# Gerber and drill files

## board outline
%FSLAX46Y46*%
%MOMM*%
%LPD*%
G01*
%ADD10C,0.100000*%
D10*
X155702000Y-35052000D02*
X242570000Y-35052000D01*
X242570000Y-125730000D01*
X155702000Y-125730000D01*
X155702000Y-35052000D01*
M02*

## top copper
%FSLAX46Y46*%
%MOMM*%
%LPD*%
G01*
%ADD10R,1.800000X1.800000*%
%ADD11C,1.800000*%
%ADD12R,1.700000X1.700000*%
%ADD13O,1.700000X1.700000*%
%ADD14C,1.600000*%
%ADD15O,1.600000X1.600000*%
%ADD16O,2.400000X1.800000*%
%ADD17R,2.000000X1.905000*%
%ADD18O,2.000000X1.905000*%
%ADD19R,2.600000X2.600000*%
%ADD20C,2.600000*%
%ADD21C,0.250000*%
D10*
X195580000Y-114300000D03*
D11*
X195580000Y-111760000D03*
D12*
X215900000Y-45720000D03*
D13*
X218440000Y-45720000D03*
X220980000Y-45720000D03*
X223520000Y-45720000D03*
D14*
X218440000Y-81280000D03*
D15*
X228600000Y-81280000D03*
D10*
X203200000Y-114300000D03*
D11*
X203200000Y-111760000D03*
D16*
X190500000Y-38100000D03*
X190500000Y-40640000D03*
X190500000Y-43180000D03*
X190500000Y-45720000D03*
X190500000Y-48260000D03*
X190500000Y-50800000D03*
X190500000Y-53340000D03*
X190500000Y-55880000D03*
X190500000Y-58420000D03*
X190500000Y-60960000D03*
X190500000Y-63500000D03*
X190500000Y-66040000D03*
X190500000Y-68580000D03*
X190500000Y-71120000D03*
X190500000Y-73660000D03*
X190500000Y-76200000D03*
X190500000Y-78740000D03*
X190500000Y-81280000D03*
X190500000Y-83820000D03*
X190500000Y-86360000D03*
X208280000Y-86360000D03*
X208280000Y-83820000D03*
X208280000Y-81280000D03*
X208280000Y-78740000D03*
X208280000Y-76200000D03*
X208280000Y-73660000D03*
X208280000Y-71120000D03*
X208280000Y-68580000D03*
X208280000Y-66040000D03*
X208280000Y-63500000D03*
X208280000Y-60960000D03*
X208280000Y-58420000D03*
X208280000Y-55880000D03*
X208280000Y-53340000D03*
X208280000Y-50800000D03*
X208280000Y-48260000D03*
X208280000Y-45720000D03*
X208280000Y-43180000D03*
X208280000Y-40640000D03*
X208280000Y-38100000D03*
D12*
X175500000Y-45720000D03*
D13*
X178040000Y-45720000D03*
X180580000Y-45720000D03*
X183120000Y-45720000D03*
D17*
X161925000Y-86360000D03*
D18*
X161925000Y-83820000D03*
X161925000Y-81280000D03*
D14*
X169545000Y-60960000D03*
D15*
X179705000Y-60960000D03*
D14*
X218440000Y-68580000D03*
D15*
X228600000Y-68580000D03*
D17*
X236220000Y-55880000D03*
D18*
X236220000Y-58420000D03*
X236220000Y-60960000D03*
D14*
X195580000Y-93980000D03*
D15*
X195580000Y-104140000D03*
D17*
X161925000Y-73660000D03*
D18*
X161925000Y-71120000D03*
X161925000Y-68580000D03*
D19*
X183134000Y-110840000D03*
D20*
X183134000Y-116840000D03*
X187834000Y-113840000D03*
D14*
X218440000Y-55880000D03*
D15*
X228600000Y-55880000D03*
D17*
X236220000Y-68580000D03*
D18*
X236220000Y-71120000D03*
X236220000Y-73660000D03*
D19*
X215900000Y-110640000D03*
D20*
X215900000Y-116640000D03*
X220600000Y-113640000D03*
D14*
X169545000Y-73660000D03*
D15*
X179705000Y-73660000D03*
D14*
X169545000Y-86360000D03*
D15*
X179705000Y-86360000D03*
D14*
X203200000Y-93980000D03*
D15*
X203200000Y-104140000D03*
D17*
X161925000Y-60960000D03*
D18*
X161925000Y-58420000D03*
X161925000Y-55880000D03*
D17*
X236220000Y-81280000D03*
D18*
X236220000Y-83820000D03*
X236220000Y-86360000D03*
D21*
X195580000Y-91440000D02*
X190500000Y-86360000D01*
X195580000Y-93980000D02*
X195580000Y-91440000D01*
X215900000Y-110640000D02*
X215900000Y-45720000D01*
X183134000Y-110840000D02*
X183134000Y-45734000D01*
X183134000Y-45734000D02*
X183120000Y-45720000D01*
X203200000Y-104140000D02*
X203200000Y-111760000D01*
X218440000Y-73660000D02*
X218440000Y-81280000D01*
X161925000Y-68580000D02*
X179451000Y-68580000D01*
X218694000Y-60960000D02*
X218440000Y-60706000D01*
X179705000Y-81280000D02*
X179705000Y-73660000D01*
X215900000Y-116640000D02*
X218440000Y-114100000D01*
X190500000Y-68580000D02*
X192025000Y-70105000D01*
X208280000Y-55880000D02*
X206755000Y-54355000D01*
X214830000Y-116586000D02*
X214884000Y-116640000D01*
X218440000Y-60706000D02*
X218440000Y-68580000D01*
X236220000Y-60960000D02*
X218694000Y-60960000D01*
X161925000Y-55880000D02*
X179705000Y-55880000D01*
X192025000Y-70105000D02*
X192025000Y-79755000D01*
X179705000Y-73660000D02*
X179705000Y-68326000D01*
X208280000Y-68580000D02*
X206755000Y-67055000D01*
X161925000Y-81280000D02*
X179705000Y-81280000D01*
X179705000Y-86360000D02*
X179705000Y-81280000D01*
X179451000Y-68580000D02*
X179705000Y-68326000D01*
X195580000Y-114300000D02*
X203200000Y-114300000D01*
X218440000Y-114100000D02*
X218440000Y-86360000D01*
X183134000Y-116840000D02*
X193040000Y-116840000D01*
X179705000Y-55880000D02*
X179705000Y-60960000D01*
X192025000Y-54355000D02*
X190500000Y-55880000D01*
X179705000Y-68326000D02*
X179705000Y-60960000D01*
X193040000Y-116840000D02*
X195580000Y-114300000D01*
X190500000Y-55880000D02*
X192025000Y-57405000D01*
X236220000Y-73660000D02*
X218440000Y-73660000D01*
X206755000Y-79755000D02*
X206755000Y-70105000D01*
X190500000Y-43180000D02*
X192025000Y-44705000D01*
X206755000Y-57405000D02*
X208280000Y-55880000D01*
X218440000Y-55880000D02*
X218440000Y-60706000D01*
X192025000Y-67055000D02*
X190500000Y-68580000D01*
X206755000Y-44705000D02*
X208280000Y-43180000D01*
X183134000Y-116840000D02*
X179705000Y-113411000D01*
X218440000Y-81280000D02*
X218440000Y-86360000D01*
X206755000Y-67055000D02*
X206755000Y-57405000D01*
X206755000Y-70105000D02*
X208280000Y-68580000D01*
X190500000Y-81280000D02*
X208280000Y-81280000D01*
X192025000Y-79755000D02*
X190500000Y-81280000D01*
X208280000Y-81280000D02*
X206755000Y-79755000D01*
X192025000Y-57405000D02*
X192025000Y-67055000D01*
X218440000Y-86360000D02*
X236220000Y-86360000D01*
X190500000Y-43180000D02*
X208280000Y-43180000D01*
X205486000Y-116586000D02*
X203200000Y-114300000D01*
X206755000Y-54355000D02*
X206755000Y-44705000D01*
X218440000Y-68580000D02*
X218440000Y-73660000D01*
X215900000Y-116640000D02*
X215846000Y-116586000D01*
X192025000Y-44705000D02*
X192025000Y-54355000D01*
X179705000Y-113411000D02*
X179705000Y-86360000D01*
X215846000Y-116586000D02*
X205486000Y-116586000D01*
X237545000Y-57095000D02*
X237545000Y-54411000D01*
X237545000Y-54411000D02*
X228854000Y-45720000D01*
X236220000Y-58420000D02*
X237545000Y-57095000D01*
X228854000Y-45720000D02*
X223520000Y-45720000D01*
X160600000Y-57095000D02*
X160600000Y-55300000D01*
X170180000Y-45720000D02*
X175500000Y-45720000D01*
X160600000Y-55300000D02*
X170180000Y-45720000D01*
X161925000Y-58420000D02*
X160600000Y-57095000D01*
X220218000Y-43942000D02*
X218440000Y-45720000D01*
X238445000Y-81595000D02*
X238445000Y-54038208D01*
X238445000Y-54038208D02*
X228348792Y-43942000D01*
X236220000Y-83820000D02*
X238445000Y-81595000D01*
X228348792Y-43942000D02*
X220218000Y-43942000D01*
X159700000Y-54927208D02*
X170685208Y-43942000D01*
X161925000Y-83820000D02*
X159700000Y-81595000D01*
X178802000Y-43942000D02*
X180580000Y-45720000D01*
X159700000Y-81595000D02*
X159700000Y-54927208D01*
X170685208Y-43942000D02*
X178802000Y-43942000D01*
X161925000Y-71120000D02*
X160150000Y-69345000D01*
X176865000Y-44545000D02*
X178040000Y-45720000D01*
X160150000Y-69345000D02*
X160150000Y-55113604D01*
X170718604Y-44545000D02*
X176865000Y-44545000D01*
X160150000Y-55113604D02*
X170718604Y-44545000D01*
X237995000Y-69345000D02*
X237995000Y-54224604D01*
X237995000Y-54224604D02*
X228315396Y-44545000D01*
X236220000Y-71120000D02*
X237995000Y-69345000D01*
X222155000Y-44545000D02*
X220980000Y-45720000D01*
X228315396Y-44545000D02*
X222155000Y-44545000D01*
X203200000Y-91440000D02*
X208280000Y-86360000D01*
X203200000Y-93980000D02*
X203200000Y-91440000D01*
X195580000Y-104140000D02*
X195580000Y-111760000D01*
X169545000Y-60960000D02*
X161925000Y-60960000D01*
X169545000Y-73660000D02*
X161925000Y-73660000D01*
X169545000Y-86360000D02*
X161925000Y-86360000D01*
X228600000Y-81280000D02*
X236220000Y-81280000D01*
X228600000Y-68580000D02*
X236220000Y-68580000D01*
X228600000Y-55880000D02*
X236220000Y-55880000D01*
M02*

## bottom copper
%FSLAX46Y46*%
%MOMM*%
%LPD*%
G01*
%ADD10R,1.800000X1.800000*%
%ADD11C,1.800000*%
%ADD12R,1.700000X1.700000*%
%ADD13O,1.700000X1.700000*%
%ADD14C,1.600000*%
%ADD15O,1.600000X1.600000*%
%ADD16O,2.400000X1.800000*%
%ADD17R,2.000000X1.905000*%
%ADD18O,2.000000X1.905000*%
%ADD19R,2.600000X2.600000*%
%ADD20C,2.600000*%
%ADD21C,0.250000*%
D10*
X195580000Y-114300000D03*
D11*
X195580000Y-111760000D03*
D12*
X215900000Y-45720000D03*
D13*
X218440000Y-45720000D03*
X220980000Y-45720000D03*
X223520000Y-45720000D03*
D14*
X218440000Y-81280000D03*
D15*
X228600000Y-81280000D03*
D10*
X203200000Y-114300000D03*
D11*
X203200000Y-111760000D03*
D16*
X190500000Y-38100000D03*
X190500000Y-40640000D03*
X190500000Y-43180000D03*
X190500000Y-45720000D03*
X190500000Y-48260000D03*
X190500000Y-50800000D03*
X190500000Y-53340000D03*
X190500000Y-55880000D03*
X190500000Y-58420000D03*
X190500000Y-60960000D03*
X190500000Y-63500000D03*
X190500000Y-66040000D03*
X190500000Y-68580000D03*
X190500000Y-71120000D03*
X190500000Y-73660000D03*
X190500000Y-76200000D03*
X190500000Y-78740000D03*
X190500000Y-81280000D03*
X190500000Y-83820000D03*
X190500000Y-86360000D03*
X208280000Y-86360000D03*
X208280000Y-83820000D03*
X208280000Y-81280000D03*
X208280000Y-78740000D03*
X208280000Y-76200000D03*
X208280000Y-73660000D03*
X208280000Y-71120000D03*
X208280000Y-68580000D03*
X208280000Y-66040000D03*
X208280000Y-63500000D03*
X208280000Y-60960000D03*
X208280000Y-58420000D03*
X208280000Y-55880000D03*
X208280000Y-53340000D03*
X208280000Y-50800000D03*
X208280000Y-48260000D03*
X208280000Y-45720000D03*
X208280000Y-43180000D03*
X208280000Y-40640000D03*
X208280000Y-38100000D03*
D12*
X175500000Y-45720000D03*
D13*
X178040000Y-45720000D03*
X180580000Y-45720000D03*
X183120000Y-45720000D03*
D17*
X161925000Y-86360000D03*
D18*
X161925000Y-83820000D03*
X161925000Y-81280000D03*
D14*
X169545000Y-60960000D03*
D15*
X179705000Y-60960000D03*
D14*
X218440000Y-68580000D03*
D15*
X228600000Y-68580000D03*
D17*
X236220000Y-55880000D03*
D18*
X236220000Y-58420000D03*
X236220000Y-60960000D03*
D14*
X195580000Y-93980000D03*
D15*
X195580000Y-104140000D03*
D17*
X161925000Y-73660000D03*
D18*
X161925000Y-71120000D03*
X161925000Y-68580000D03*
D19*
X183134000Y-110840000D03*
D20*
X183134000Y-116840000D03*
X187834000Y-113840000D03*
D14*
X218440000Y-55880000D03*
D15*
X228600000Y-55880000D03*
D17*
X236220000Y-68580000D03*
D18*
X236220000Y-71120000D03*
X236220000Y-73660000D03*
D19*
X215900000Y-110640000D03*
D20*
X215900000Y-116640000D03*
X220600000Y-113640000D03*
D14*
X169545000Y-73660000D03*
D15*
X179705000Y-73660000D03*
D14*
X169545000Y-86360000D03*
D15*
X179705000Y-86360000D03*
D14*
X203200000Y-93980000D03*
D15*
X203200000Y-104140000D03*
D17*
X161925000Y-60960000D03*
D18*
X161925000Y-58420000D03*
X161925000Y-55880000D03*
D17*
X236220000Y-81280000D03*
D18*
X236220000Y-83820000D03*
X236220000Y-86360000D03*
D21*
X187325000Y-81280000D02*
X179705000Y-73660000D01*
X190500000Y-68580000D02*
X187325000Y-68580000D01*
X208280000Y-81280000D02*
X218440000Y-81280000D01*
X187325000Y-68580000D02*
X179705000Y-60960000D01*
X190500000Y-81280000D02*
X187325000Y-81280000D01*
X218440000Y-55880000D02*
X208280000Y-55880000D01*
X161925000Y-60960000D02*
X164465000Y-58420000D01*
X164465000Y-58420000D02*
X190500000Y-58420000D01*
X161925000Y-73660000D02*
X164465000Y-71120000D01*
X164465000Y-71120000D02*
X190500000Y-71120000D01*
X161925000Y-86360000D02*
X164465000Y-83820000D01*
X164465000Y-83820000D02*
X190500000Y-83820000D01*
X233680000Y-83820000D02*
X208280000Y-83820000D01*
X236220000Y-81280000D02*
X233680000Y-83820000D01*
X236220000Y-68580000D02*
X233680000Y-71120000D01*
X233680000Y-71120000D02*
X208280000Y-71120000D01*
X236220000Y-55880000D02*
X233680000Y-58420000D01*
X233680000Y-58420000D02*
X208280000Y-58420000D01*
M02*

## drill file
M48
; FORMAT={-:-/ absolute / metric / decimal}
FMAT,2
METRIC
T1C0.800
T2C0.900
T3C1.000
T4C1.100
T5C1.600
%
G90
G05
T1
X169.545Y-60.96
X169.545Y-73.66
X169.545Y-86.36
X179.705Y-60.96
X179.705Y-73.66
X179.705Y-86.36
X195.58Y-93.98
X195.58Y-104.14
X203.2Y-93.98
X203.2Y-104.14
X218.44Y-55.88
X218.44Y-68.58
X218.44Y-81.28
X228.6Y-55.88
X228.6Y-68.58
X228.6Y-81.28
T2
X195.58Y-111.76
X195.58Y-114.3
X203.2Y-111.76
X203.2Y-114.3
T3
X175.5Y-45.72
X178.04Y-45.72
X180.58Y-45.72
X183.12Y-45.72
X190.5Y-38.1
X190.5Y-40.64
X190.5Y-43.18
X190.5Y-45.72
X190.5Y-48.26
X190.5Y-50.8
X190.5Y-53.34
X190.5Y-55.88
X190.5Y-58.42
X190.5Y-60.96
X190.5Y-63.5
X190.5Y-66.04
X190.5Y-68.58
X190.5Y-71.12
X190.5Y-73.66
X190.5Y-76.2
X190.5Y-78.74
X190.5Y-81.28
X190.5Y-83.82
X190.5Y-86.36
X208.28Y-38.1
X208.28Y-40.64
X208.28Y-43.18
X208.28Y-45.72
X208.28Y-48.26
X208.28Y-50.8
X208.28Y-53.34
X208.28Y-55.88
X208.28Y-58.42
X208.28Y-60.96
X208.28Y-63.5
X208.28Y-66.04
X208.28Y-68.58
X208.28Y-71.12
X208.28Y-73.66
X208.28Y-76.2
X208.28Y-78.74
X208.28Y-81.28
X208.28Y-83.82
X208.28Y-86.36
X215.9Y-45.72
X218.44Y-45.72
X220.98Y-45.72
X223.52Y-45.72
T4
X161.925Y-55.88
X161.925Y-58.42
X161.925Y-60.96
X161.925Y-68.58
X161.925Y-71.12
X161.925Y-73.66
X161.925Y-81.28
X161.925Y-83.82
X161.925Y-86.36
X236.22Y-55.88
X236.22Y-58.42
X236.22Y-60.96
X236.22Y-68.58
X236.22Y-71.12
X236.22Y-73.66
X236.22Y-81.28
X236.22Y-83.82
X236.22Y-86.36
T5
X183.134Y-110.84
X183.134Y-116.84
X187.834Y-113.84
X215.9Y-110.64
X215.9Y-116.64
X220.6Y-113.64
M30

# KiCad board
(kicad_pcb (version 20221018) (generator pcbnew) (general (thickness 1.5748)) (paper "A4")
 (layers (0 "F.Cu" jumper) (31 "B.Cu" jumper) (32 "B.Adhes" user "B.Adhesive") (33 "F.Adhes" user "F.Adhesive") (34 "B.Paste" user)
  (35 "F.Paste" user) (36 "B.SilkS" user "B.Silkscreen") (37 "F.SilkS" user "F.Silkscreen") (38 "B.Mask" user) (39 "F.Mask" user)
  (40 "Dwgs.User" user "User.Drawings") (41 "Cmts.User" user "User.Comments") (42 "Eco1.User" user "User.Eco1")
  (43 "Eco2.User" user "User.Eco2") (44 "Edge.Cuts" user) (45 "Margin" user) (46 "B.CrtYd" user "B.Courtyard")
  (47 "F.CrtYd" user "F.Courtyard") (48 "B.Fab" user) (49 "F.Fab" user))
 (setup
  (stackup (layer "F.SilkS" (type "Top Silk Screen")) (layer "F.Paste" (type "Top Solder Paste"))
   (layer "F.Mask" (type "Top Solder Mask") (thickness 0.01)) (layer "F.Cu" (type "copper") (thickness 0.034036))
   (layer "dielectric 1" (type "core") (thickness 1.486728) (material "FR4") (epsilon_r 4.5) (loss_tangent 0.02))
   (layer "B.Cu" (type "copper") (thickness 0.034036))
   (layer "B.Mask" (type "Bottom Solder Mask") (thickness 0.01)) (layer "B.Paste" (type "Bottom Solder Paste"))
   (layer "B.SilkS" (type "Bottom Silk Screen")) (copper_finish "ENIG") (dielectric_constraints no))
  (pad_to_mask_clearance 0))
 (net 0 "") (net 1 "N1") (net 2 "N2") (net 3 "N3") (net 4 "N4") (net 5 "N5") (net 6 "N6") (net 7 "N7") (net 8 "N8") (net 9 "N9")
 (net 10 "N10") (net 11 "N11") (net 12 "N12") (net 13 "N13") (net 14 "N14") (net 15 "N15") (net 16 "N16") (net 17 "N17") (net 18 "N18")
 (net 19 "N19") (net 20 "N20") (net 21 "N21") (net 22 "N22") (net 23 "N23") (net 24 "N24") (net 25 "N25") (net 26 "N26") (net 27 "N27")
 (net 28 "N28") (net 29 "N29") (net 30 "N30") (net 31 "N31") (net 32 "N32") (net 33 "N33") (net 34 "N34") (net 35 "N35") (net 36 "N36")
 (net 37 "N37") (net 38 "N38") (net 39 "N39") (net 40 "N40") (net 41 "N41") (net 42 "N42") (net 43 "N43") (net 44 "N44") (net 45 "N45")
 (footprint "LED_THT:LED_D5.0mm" (layer "F.Cu") (at 195.58 114.3 90)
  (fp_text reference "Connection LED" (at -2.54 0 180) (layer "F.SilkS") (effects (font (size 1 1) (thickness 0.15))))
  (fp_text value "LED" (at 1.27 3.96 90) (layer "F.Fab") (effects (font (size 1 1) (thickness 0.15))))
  (pad "1" thru_hole rect (at 0 0 90) (size 1.8 1.8) (drill 0.9) (layers "*.Cu" "*.Mask") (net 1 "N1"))
  (pad "2" thru_hole circle (at 2.54 0 90) (size 1.8 1.8) (drill 0.9) (layers "*.Cu" "*.Mask") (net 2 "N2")))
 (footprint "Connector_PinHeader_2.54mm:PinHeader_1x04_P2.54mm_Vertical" (layer "F.Cu") (at 215.9 45.72 90)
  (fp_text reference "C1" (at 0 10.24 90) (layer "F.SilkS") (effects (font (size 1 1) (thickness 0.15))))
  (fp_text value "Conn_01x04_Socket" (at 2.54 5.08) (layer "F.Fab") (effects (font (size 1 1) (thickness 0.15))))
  (pad "1" thru_hole rect (at 0 0 90) (size 1.7 1.7) (drill 1) (layers "*.Cu" "*.Mask") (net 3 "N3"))
  (pad "2" thru_hole oval (at 0 2.54 90) (size 1.7 1.7) (drill 1) (layers "*.Cu" "*.Mask") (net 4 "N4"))
  (pad "3" thru_hole oval (at 0 5.08 90) (size 1.7 1.7) (drill 1) (layers "*.Cu" "*.Mask") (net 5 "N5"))
  (pad "4" thru_hole oval (at 0 7.62 90) (size 1.7 1.7) (drill 1) (layers "*.Cu" "*.Mask") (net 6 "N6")))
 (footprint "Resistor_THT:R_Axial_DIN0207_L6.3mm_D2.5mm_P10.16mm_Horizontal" (layer "F.Cu") (at 218.44 81.28)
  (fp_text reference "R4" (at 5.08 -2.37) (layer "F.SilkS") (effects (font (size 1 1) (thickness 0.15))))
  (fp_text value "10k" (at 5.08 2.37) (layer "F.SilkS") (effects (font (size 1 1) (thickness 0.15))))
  (pad "1" thru_hole circle (at 0 0) (size 1.6 1.6) (drill 0.8) (layers "*.Cu" "*.Mask") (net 1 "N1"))
  (pad "2" thru_hole oval (at 10.16 0) (size 1.6 1.6) (drill 0.8) (layers "*.Cu" "*.Mask") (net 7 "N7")))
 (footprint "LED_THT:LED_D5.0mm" (layer "F.Cu") (at 203.2 114.3 90)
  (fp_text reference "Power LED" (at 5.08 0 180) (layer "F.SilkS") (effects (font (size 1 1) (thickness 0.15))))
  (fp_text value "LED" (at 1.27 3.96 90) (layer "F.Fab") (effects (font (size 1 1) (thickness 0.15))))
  (pad "1" thru_hole rect (at 0 0 90) (size 1.8 1.8) (drill 0.9) (layers "*.Cu" "*.Mask") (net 1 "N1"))
  (pad "2" thru_hole circle (at 2.54 0 90) (size 1.8 1.8) (drill 0.9) (layers "*.Cu" "*.Mask") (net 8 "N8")))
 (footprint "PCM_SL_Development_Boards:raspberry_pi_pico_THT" (layer "F.Cu") (at 190.5 38.1)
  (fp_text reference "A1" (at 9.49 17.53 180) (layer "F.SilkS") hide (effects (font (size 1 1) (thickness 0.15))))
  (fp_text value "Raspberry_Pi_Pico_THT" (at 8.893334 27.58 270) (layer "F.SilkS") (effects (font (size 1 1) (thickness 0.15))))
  (pad "1" thru_hole oval (at 0 0 270) (size 1.8 2.4) (drill 1) (layers "*.Cu" "*.Mask") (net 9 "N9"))
  (pad "2" thru_hole oval (at 0 2.54 270) (size 1.8 2.4) (drill 1) (layers "*.Cu" "*.Mask") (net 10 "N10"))
  (pad "3" thru_hole oval (at 0 5.08 270) (size 1.8 2.4) (drill 1) (layers "*.Cu" "*.Mask") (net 1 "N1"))
  (pad "4" thru_hole oval (at 0 7.62 270) (size 1.8 2.4) (drill 1) (layers "*.Cu" "*.Mask") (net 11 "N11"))
  (pad "5" thru_hole oval (at 0 10.16 270) (size 1.8 2.4) (drill 1) (layers "*.Cu" "*.Mask") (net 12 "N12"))
  (pad "6" thru_hole oval (at 0 12.7 270) (size 1.8 2.4) (drill 1) (layers "*.Cu" "*.Mask") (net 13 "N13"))
  (pad "7" thru_hole oval (at 0 15.24 270) (size 1.8 2.4) (drill 1) (layers "*.Cu" "*.Mask") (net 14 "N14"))
  (pad "8" thru_hole oval (at 0 17.78 270) (size 1.8 2.4) (drill 1) (layers "*.Cu" "*.Mask") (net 1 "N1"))
  (pad "9" thru_hole oval (at 0 20.32 270) (size 1.8 2.4) (drill 1) (layers "*.Cu" "*.Mask") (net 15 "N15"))
  (pad "10" thru_hole oval (at 0 22.86 270) (size 1.8 2.4) (drill 1) (layers "*.Cu" "*.Mask") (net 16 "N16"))
  (pad "11" thru_hole oval (at 0 25.4 270) (size 1.8 2.4) (drill 1) (layers "*.Cu" "*.Mask") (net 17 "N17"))
  (pad "12" thru_hole oval (at 0 27.94 270) (size 1.8 2.4) (drill 1) (layers "*.Cu" "*.Mask") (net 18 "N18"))
  (pad "13" thru_hole oval (at 0 30.48 270) (size 1.8 2.4) (drill 1) (layers "*.Cu" "*.Mask") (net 1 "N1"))
  (pad "14" thru_hole oval (at 0 33.02 270) (size 1.8 2.4) (drill 1) (layers "*.Cu" "*.Mask") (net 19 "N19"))
  (pad "15" thru_hole oval (at 0 35.56 270) (size 1.8 2.4) (drill 1) (layers "*.Cu" "*.Mask") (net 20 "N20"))
  (pad "16" thru_hole oval (at 0 38.1 270) (size 1.8 2.4) (drill 1) (layers "*.Cu" "*.Mask") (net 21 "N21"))
  (pad "17" thru_hole oval (at 0 40.64 270) (size 1.8 2.4) (drill 1) (layers "*.Cu" "*.Mask") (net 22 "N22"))
  (pad "18" thru_hole oval (at 0 43.18 270) (size 1.8 2.4) (drill 1) (layers "*.Cu" "*.Mask") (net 1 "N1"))
  (pad "19" thru_hole oval (at 0 45.72 270) (size 1.8 2.4) (drill 1) (layers "*.Cu" "*.Mask") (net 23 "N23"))
  (pad "20" thru_hole oval (at 0 48.26 270) (size 1.8 2.4) (drill 1) (layers "*.Cu" "*.Mask") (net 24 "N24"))
  (pad "21" thru_hole oval (at 17.78 48.26 270) (size 1.8 2.4) (drill 1) (layers "*.Cu" "*.Mask") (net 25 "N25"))
  (pad "22" thru_hole oval (at 17.78 45.72 270) (size 1.8 2.4) (drill 1) (layers "*.Cu" "*.Mask") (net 7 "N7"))
  (pad "23" thru_hole oval (at 17.78 43.18 270) (size 1.8 2.4) (drill 1) (layers "*.Cu" "*.Mask") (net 1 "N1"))
  (pad "24" thru_hole oval (at 17.78 40.64 270) (size 1.8 2.4) (drill 1) (layers "*.Cu" "*.Mask") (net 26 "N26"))
  (pad "25" thru_hole oval (at 17.78 38.1 270) (size 1.8 2.4) (drill 1) (layers "*.Cu" "*.Mask") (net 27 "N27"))
  (pad "26" thru_hole oval (at 17.78 35.56 270) (size 1.8 2.4) (drill 1) (layers "*.Cu" "*.Mask") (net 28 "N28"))
  (pad "27" thru_hole oval (at 17.78 33.02 270) (size 1.8 2.4) (drill 1) (layers "*.Cu" "*.Mask") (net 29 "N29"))
  (pad "28" thru_hole oval (at 17.78 30.48 270) (size 1.8 2.4) (drill 1) (layers "*.Cu" "*.Mask") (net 1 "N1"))
  (pad "29" thru_hole oval (at 17.78 27.94 270) (size 1.8 2.4) (drill 1) (layers "*.Cu" "*.Mask") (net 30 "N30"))
  (pad "30" thru_hole oval (at 17.78 25.4 270) (size 1.8 2.4) (drill 1) (layers "*.Cu" "*.Mask") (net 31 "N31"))
  (pad "31" thru_hole oval (at 17.78 22.86 270) (size 1.8 2.4) (drill 1) (layers "*.Cu" "*.Mask") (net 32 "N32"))
  (pad "32" thru_hole oval (at 17.78 20.32 270) (size 1.8 2.4) (drill 1) (layers "*.Cu" "*.Mask") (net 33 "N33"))
  (pad "33" thru_hole oval (at 17.78 17.78 270) (size 1.8 2.4) (drill 1) (layers "*.Cu" "*.Mask") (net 1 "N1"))
  (pad "34" thru_hole oval (at 17.78 15.24 270) (size 1.8 2.4) (drill 1) (layers "*.Cu" "*.Mask") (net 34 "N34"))
  (pad "35" thru_hole oval (at 17.78 12.7 270) (size 1.8 2.4) (drill 1) (layers "*.Cu" "*.Mask") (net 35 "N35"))
  (pad "36" thru_hole oval (at 17.78 10.16 270) (size 1.8 2.4) (drill 1) (layers "*.Cu" "*.Mask") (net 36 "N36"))
  (pad "37" thru_hole oval (at 17.78 7.62 270) (size 1.8 2.4) (drill 1) (layers "*.Cu" "*.Mask") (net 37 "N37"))
  (pad "38" thru_hole oval (at 17.78 5.08 270) (size 1.8 2.4) (drill 1) (layers "*.Cu" "*.Mask") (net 1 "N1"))
  (pad "39" thru_hole oval (at 17.78 2.54 270) (size 1.8 2.4) (drill 1) (layers "*.Cu" "*.Mask") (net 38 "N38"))
  (pad "40" thru_hole oval (at 17.78 0 270) (size 1.8 2.4) (drill 1) (layers "*.Cu" "*.Mask") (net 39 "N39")))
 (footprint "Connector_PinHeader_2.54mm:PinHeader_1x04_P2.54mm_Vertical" (layer "F.Cu") (at 175.5 45.72 90)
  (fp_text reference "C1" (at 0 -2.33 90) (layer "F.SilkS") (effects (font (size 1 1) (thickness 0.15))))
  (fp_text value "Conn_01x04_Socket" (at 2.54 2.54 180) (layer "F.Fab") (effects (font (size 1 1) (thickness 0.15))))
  (pad "1" thru_hole rect (at 0 0 90) (size 1.7 1.7) (drill 1) (layers "*.Cu" "*.Mask") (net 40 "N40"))
  (pad "2" thru_hole oval (at 0 2.54 90) (size 1.7 1.7) (drill 1) (layers "*.Cu" "*.Mask") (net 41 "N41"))
  (pad "3" thru_hole oval (at 0 5.08 90) (size 1.7 1.7) (drill 1) (layers "*.Cu" "*.Mask") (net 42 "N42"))
  (pad "4" thru_hole oval (at 0 7.62 90) (size 1.7 1.7) (drill 1) (layers "*.Cu" "*.Mask") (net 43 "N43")))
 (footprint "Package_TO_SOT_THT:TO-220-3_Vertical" (layer "F.Cu") (at 161.925 86.36 90)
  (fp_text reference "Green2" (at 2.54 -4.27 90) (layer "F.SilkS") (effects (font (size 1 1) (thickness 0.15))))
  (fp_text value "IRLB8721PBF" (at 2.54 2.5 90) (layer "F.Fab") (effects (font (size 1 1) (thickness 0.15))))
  (pad "1" thru_hole rect (at 0 0 90) (size 1.905 2) (drill 1.1) (layers "*.Cu" "*.Mask") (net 23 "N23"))
  (pad "2" thru_hole oval (at 2.54 0 90) (size 1.905 2) (drill 1.1) (layers "*.Cu" "*.Mask") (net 42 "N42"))
  (pad "3" thru_hole oval (at 5.08 0 90) (size 1.905 2) (drill 1.1) (layers "*.Cu" "*.Mask") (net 1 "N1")))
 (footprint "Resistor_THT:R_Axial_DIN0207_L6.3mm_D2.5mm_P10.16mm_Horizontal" (layer "F.Cu") (at 169.545 60.96)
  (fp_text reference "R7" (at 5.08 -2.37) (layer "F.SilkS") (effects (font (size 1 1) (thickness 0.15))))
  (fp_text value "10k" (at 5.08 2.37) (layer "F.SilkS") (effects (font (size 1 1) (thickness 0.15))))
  (pad "1" thru_hole circle (at 0 0) (size 1.6 1.6) (drill 0.8) (layers "*.Cu" "*.Mask") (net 15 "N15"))
  (pad "2" thru_hole oval (at 10.16 0) (size 1.6 1.6) (drill 0.8) (layers "*.Cu" "*.Mask") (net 1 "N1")))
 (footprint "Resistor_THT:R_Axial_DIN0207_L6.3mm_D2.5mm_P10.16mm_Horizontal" (layer "F.Cu") (at 218.44 68.58)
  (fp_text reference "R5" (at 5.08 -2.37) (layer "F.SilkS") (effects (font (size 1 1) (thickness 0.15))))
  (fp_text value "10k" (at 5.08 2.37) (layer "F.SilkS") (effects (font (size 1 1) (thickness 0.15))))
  (pad "1" thru_hole circle (at 0 0) (size 1.6 1.6) (drill 0.8) (layers "*.Cu" "*.Mask") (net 1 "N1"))
  (pad "2" thru_hole oval (at 10.16 0) (size 1.6 1.6) (drill 0.8) (layers "*.Cu" "*.Mask") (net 29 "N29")))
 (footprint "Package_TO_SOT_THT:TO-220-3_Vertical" (layer "F.Cu") (at 236.22 55.88 -90)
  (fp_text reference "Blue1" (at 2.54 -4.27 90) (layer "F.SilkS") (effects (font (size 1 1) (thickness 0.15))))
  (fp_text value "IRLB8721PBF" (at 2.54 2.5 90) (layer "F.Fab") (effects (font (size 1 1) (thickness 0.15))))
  (pad "1" thru_hole rect (at 0 0 270) (size 1.905 2) (drill 1.1) (layers "*.Cu" "*.Mask") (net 33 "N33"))
  (pad "2" thru_hole oval (at 2.54 0 270) (size 1.905 2) (drill 1.1) (layers "*.Cu" "*.Mask") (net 6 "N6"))
  (pad "3" thru_hole oval (at 5.08 0 270) (size 1.905 2) (drill 1.1) (layers "*.Cu" "*.Mask") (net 1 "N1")))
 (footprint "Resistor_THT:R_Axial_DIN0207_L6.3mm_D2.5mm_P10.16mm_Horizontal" (layer "F.Cu") (at 195.58 93.98 -90)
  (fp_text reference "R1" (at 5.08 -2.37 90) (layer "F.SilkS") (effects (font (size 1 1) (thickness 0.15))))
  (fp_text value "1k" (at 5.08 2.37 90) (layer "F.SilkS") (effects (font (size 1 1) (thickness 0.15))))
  (pad "1" thru_hole circle (at 0 0 270) (size 1.6 1.6) (drill 0.8) (layers "*.Cu" "*.Mask") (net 24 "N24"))
  (pad "2" thru_hole oval (at 10.16 0 270) (size 1.6 1.6) (drill 0.8) (layers "*.Cu" "*.Mask") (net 2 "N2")))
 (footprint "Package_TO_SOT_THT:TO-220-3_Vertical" (layer "F.Cu") (at 161.925 73.66 90)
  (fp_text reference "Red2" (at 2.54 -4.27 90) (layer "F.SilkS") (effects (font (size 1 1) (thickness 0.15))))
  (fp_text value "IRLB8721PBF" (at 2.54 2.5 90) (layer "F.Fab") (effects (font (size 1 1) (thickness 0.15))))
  (pad "1" thru_hole rect (at 0 0 90) (size 1.905 2) (drill 1.1) (layers "*.Cu" "*.Mask") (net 19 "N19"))
  (pad "2" thru_hole oval (at 2.54 0 90) (size 1.905 2) (drill 1.1) (layers "*.Cu" "*.Mask") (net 41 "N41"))
  (pad "3" thru_hole oval (at 5.08 0 90) (size 1.905 2) (drill 1.1) (layers "*.Cu" "*.Mask") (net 1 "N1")))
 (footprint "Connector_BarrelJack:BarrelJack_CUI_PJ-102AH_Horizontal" (layer "F.Cu") (at 183.134 110.84)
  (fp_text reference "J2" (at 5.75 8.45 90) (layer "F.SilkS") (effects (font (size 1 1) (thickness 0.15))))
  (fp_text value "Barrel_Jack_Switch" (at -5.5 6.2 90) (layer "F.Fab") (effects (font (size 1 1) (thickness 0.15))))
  (pad "1" thru_hole rect (at 0 0) (size 2.6 2.6) (drill 1.6) (layers "*.Cu" "*.Mask") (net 43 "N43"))
  (pad "2" thru_hole circle (at 0 6) (size 2.6 2.6) (drill 1.6) (layers "*.Cu" "*.Mask") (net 1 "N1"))
  (pad "3" thru_hole circle (at 4.7 3) (size 2.6 2.6) (drill 1.6) (layers "*.Cu" "*.Mask") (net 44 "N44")))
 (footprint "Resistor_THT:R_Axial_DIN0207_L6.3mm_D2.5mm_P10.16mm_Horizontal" (layer "F.Cu") (at 218.44 55.88)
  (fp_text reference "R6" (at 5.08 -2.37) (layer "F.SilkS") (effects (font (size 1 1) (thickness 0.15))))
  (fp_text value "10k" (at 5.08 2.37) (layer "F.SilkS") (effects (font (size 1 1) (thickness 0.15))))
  (pad "1" thru_hole circle (at 0 0) (size 1.6 1.6) (drill 0.8) (layers "*.Cu" "*.Mask") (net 1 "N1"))
  (pad "2" thru_hole oval (at 10.16 0) (size 1.6 1.6) (drill 0.8) (layers "*.Cu" "*.Mask") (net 33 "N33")))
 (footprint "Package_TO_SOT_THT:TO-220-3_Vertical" (layer "F.Cu") (at 236.22 68.58 -90)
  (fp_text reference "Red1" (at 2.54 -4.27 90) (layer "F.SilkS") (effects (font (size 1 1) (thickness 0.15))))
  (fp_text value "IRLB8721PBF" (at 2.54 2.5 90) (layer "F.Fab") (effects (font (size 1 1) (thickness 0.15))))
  (pad "1" thru_hole rect (at 0 0 270) (size 1.905 2) (drill 1.1) (layers "*.Cu" "*.Mask") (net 29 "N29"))
  (pad "2" thru_hole oval (at 2.54 0 270) (size 1.905 2) (drill 1.1) (layers "*.Cu" "*.Mask") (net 5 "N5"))
  (pad "3" thru_hole oval (at 5.08 0 270) (size 1.905 2) (drill 1.1) (layers "*.Cu" "*.Mask") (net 1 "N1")))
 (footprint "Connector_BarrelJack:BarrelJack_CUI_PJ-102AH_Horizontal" (layer "F.Cu") (at 215.9 110.64)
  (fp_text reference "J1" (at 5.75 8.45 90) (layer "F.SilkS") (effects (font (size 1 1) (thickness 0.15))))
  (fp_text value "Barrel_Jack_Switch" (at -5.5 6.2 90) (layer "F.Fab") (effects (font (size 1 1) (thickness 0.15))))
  (pad "1" thru_hole rect (at 0 0) (size 2.6 2.6) (drill 1.6) (layers "*.Cu" "*.Mask") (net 3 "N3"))
  (pad "2" thru_hole circle (at 0 6) (size 2.6 2.6) (drill 1.6) (layers "*.Cu" "*.Mask") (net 1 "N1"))
  (pad "3" thru_hole circle (at 4.7 3) (size 2.6 2.6) (drill 1.6) (layers "*.Cu" "*.Mask") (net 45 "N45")))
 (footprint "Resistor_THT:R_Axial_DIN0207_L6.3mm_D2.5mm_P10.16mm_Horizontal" (layer "F.Cu") (at 169.545 73.66)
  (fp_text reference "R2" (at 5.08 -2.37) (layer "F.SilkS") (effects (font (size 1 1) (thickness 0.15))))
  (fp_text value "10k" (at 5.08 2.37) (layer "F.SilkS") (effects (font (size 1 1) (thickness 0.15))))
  (pad "1" thru_hole circle (at 0 0) (size 1.6 1.6) (drill 0.8) (layers "*.Cu" "*.Mask") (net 19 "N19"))
  (pad "2" thru_hole oval (at 10.16 0) (size 1.6 1.6) (drill 0.8) (layers "*.Cu" "*.Mask") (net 1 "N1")))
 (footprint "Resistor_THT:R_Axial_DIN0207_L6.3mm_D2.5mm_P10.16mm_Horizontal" (layer "F.Cu") (at 169.545 86.36)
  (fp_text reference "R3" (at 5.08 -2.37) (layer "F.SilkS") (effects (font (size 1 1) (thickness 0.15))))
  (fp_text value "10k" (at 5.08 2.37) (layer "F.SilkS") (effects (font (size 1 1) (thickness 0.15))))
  (pad "1" thru_hole circle (at 0 0) (size 1.6 1.6) (drill 0.8) (layers "*.Cu" "*.Mask") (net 23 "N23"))
  (pad "2" thru_hole oval (at 10.16 0) (size 1.6 1.6) (drill 0.8) (layers "*.Cu" "*.Mask") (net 1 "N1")))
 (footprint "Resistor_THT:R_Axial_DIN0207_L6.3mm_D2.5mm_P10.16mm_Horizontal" (layer "F.Cu") (at 203.2 93.98 -90)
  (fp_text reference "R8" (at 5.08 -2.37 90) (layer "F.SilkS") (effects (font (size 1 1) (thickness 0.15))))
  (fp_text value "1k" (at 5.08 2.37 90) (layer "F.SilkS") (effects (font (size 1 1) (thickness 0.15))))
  (pad "1" thru_hole circle (at 0 0 270) (size 1.6 1.6) (drill 0.8) (layers "*.Cu" "*.Mask") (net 25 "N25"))
  (pad "2" thru_hole oval (at 10.16 0 270) (size 1.6 1.6) (drill 0.8) (layers "*.Cu" "*.Mask") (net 8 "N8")))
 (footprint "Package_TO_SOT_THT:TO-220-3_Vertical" (layer "F.Cu") (at 161.925 60.96 90)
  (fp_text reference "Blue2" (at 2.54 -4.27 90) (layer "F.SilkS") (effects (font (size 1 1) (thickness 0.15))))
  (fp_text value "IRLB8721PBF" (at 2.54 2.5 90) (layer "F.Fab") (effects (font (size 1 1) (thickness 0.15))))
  (pad "1" thru_hole rect (at 0 0 90) (size 1.905 2) (drill 1.1) (layers "*.Cu" "*.Mask") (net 15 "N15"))
  (pad "2" thru_hole oval (at 2.54 0 90) (size 1.905 2) (drill 1.1) (layers "*.Cu" "*.Mask") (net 40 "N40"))
  (pad "3" thru_hole oval (at 5.08 0 90) (size 1.905 2) (drill 1.1) (layers "*.Cu" "*.Mask") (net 1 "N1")))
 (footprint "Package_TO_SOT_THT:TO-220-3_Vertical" (layer "F.Cu") (at 236.22 81.28 -90)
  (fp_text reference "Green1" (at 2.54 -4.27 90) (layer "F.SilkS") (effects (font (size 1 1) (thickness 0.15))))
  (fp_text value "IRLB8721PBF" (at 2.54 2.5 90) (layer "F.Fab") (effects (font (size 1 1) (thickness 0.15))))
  (pad "1" thru_hole rect (at 0 0 270) (size 1.905 2) (drill 1.1) (layers "*.Cu" "*.Mask") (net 7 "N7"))
  (pad "2" thru_hole oval (at 2.54 0 270) (size 1.905 2) (drill 1.1) (layers "*.Cu" "*.Mask") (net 4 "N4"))
  (pad "3" thru_hole oval (at 5.08 0 270) (size 1.905 2) (drill 1.1) (layers "*.Cu" "*.Mask") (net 1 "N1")))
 (gr_rect (start 155.702 35.052) (end 242.57 125.73) (stroke (width 0.1) (type default)) (fill none) (layer "Edge.Cuts"))
 (segment (start 195.58 91.44) (end 190.5 86.36) (width 0.25) (layer "F.Cu") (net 24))
 (segment (start 195.58 93.98) (end 195.58 91.44) (width 0.25) (layer "F.Cu") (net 24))
 (segment (start 215.9 110.64) (end 215.9 45.72) (width 0.25) (layer "F.Cu") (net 3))
 (segment (start 183.134 110.84) (end 183.134 45.734) (width 0.25) (layer "F.Cu") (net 43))
 (segment (start 183.134 45.734) (end 183.12 45.72) (width 0.25) (layer "F.Cu") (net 43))
 (segment (start 203.2 104.14) (end 203.2 111.76) (width 0.25) (layer "F.Cu") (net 8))
 (segment (start 218.44 73.66) (end 218.44 81.28) (width 0.25) (layer "F.Cu") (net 1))
 (segment (start 161.925 68.58) (end 179.451 68.58) (width 0.25) (layer "F.Cu") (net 1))
 (segment (start 218.694 60.96) (end 218.44 60.706) (width 0.25) (layer "F.Cu") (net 1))
 (segment (start 179.705 81.28) (end 179.705 73.66) (width 0.25) (layer "F.Cu") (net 1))
 (segment (start 215.9 116.64) (end 218.44 114.1) (width 0.25) (layer "F.Cu") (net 1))
 (segment (start 190.5 68.58) (end 192.025 70.105) (width 0.25) (layer "F.Cu") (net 1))
 (segment (start 208.28 55.88) (end 206.755 54.355) (width 0.25) (layer "F.Cu") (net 1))
 (segment (start 214.83 116.586) (end 214.884 116.64) (width 0.25) (layer "F.Cu") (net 1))
 (segment (start 218.44 60.706) (end 218.44 68.58) (width 0.25) (layer "F.Cu") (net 1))
 (segment (start 236.22 60.96) (end 218.694 60.96) (width 0.25) (layer "F.Cu") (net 1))
 (segment (start 161.925 55.88) (end 179.705 55.88) (width 0.25) (layer "F.Cu") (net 1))
 (segment (start 192.025 70.105) (end 192.025 79.755) (width 0.25) (layer "F.Cu") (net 1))
 (segment (start 179.705 73.66) (end 179.705 68.326) (width 0.25) (layer "F.Cu") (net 1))
 (segment (start 208.28 68.58) (end 206.755 67.055) (width 0.25) (layer "F.Cu") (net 1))
 (segment (start 161.925 81.28) (end 179.705 81.28) (width 0.25) (layer "F.Cu") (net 1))
 (segment (start 179.705 86.36) (end 179.705 81.28) (width 0.25) (layer "F.Cu") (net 1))
 (segment (start 179.451 68.58) (end 179.705 68.326) (width 0.25) (layer "F.Cu") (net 1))
 (segment (start 195.58 114.3) (end 203.2 114.3) (width 0.25) (layer "F.Cu") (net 1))
 (segment (start 218.44 114.1) (end 218.44 86.36) (width 0.25) (layer "F.Cu") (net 1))
 (segment (start 183.134 116.84) (end 193.04 116.84) (width 0.25) (layer "F.Cu") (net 1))
 (segment (start 179.705 55.88) (end 179.705 60.96) (width 0.25) (layer "F.Cu") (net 1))
 (segment (start 192.025 54.355) (end 190.5 55.88) (width 0.25) (layer "F.Cu") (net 1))
 (segment (start 179.705 68.326) (end 179.705 60.96) (width 0.25) (layer "F.Cu") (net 1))
 (segment (start 193.04 116.84) (end 195.58 114.3) (width 0.25) (layer "F.Cu") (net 1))
 (segment (start 190.5 55.88) (end 192.025 57.405) (width 0.25) (layer "F.Cu") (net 1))
 (segment (start 236.22 73.66) (end 218.44 73.66) (width 0.25) (layer "F.Cu") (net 1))
 (segment (start 206.755 79.755) (end 206.755 70.105) (width 0.25) (layer "F.Cu") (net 1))
 (segment (start 190.5 43.18) (end 192.025 44.705) (width 0.25) (layer "F.Cu") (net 1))
 (segment (start 206.755 57.405) (end 208.28 55.88) (width 0.25) (layer "F.Cu") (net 1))
 (segment (start 218.44 55.88) (end 218.44 60.706) (width 0.25) (layer "F.Cu") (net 1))
 (segment (start 192.025 67.055) (end 190.5 68.58) (width 0.25) (layer "F.Cu") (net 1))
 (segment (start 206.755 44.705) (end 208.28 43.18) (width 0.25) (layer "F.Cu") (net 1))
 (segment (start 183.134 116.84) (end 179.705 113.411) (width 0.25) (layer "F.Cu") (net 1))
 (segment (start 218.44 81.28) (end 218.44 86.36) (width 0.25) (layer "F.Cu") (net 1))
 (segment (start 206.755 67.055) (end 206.755 57.405) (width 0.25) (layer "F.Cu") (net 1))
 (segment (start 206.755 70.105) (end 208.28 68.58) (width 0.25) (layer "F.Cu") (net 1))
 (segment (start 190.5 81.28) (end 208.28 81.28) (width 0.25) (layer "F.Cu") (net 1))
 (segment (start 192.025 79.755) (end 190.5 81.28) (width 0.25) (layer "F.Cu") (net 1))
 (segment (start 208.28 81.28) (end 206.755 79.755) (width 0.25) (layer "F.Cu") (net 1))
 (segment (start 192.025 57.405) (end 192.025 67.055) (width 0.25) (layer "F.Cu") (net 1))
 (segment (start 218.44 86.36) (end 236.22 86.36) (width 0.25) (layer "F.Cu") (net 1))
 (segment (start 190.5 43.18) (end 208.28 43.18) (width 0.25) (layer "F.Cu") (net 1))
 (segment (start 205.486 116.586) (end 203.2 114.3) (width 0.25) (layer "F.Cu") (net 1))
 (segment (start 206.755 54.355) (end 206.755 44.705) (width 0.25) (layer "F.Cu") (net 1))
 (segment (start 218.44 68.58) (end 218.44 73.66) (width 0.25) (layer "F.Cu") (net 1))
 (segment (start 215.9 116.64) (end 215.846 116.586) (width 0.25) (layer "F.Cu") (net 1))
 (segment (start 192.025 44.705) (end 192.025 54.355) (width 0.25) (layer "F.Cu") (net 1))
 (segment (start 179.705 113.411) (end 179.705 86.36) (width 0.25) (layer "F.Cu") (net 1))
 (segment (start 215.846 116.586) (end 205.486 116.586) (width 0.25) (layer "F.Cu") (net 1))
 (segment (start 187.325 81.28) (end 179.705 73.66) (width 0.25) (layer "B.Cu") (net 1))
 (segment (start 190.5 68.58) (end 187.325 68.58) (width 0.25) (layer "B.Cu") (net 1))
 (segment (start 208.28 81.28) (end 218.44 81.28) (width 0.25) (layer "B.Cu") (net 1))
 (segment (start 187.325 68.58) (end 179.705 60.96) (width 0.25) (layer "B.Cu") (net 1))
 (segment (start 190.5 81.28) (end 187.325 81.28) (width 0.25) (layer "B.Cu") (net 1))
 (segment (start 218.44 55.88) (end 208.28 55.88) (width 0.25) (layer "B.Cu") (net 1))
 (segment (start 237.545 57.095) (end 237.545 54.411) (width 0.25) (layer "F.Cu") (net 6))
 (segment (start 237.545 54.411) (end 228.854 45.72) (width 0.25) (layer "F.Cu") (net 6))
 (segment (start 236.22 58.42) (end 237.545 57.095) (width 0.25) (layer "F.Cu") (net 6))
 (segment (start 228.854 45.72) (end 223.52 45.72) (width 0.25) (layer "F.Cu") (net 6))
 (segment (start 160.6 57.095) (end 160.6 55.3) (width 0.25) (layer "F.Cu") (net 40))
 (segment (start 170.18 45.72) (end 175.5 45.72) (width 0.25) (layer "F.Cu") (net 40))
 (segment (start 160.6 55.3) (end 170.18 45.72) (width 0.25) (layer "F.Cu") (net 40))
 (segment (start 161.925 58.42) (end 160.6 57.095) (width 0.25) (layer "F.Cu") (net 40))
 (segment (start 220.218 43.942) (end 218.44 45.72) (width 0.25) (layer "F.Cu") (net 4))
 (segment (start 238.445 81.595) (end 238.445 54.038208) (width 0.25) (layer "F.Cu") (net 4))
 (segment (start 238.445 54.038208) (end 228.348792 43.942) (width 0.25) (layer "F.Cu") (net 4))
 (segment (start 236.22 83.82) (end 238.445 81.595) (width 0.25) (layer "F.Cu") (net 4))
 (segment (start 228.348792 43.942) (end 220.218 43.942) (width 0.25) (layer "F.Cu") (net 4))
 (segment (start 159.7 54.927208) (end 170.685208 43.942) (width 0.25) (layer "F.Cu") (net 42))
 (segment (start 161.925 83.82) (end 159.7 81.595) (width 0.25) (layer "F.Cu") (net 42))
 (segment (start 178.802 43.942) (end 180.58 45.72) (width 0.25) (layer "F.Cu") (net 42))
 (segment (start 159.7 81.595) (end 159.7 54.927208) (width 0.25) (layer "F.Cu") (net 42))
 (segment (start 170.685208 43.942) (end 178.802 43.942) (width 0.25) (layer "F.Cu") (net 42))
 (segment (start 161.925 71.12) (end 160.15 69.345) (width 0.25) (layer "F.Cu") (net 41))
 (segment (start 176.865 44.545) (end 178.04 45.72) (width 0.25) (layer "F.Cu") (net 41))
 (segment (start 160.15 69.345) (end 160.15 55.113604) (width 0.25) (layer "F.Cu") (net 41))
 (segment (start 170.718604 44.545) (end 176.865 44.545) (width 0.25) (layer "F.Cu") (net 41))
 (segment (start 160.15 55.113604) (end 170.718604 44.545) (width 0.25) (layer "F.Cu") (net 41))
 (segment (start 237.995 69.345) (end 237.995 54.224604) (width 0.25) (layer "F.Cu") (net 5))
 (segment (start 237.995 54.224604) (end 228.315396 44.545) (width 0.25) (layer "F.Cu") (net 5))
 (segment (start 236.22 71.12) (end 237.995 69.345) (width 0.25) (layer "F.Cu") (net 5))
 (segment (start 222.155 44.545) (end 220.98 45.72) (width 0.25) (layer "F.Cu") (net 5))
 (segment (start 228.315396 44.545) (end 222.155 44.545) (width 0.25) (layer "F.Cu") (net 5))
 (segment (start 203.2 91.44) (end 208.28 86.36) (width 0.25) (layer "F.Cu") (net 25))
 (segment (start 203.2 93.98) (end 203.2 91.44) (width 0.25) (layer "F.Cu") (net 25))
 (segment (start 195.58 104.14) (end 195.58 111.76) (width 0.25) (layer "F.Cu") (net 2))
 (segment (start 169.545 60.96) (end 161.925 60.96) (width 0.25) (layer "F.Cu") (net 15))
 (segment (start 161.925 60.96) (end 164.465 58.42) (width 0.25) (layer "B.Cu") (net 15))
 (segment (start 164.465 58.42) (end 190.5 58.42) (width 0.25) (layer "B.Cu") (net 15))
 (segment (start 169.545 73.66) (end 161.925 73.66) (width 0.25) (layer "F.Cu") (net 19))
 (segment (start 161.925 73.66) (end 164.465 71.12) (width 0.25) (layer "B.Cu") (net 19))
 (segment (start 164.465 71.12) (end 190.5 71.12) (width 0.25) (layer "B.Cu") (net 19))
 (segment (start 169.545 86.36) (end 161.925 86.36) (width 0.25) (layer "F.Cu") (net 23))
 (segment (start 161.925 86.36) (end 164.465 83.82) (width 0.25) (layer "B.Cu") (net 23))
 (segment (start 164.465 83.82) (end 190.5 83.82) (width 0.25) (layer "B.Cu") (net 23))
 (segment (start 228.6 81.28) (end 236.22 81.28) (width 0.25) (layer "F.Cu") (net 7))
 (segment (start 233.68 83.82) (end 208.28 83.82) (width 0.25) (layer "B.Cu") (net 7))
 (segment (start 236.22 81.28) (end 233.68 83.82) (width 0.25) (layer "B.Cu") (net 7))
 (segment (start 228.6 68.58) (end 236.22 68.58) (width 0.25) (layer "F.Cu") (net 29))
 (segment (start 236.22 68.58) (end 233.68 71.12) (width 0.25) (layer "B.Cu") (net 29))
 (segment (start 233.68 71.12) (end 208.28 71.12) (width 0.25) (layer "B.Cu") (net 29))
 (segment (start 228.6 55.88) (end 236.22 55.88) (width 0.25) (layer "F.Cu") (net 33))
 (segment (start 236.22 55.88) (end 233.68 58.42) (width 0.25) (layer "B.Cu") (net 33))
 (segment (start 233.68 58.42) (end 208.28 58.42) (width 0.25) (layer "B.Cu") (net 33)))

